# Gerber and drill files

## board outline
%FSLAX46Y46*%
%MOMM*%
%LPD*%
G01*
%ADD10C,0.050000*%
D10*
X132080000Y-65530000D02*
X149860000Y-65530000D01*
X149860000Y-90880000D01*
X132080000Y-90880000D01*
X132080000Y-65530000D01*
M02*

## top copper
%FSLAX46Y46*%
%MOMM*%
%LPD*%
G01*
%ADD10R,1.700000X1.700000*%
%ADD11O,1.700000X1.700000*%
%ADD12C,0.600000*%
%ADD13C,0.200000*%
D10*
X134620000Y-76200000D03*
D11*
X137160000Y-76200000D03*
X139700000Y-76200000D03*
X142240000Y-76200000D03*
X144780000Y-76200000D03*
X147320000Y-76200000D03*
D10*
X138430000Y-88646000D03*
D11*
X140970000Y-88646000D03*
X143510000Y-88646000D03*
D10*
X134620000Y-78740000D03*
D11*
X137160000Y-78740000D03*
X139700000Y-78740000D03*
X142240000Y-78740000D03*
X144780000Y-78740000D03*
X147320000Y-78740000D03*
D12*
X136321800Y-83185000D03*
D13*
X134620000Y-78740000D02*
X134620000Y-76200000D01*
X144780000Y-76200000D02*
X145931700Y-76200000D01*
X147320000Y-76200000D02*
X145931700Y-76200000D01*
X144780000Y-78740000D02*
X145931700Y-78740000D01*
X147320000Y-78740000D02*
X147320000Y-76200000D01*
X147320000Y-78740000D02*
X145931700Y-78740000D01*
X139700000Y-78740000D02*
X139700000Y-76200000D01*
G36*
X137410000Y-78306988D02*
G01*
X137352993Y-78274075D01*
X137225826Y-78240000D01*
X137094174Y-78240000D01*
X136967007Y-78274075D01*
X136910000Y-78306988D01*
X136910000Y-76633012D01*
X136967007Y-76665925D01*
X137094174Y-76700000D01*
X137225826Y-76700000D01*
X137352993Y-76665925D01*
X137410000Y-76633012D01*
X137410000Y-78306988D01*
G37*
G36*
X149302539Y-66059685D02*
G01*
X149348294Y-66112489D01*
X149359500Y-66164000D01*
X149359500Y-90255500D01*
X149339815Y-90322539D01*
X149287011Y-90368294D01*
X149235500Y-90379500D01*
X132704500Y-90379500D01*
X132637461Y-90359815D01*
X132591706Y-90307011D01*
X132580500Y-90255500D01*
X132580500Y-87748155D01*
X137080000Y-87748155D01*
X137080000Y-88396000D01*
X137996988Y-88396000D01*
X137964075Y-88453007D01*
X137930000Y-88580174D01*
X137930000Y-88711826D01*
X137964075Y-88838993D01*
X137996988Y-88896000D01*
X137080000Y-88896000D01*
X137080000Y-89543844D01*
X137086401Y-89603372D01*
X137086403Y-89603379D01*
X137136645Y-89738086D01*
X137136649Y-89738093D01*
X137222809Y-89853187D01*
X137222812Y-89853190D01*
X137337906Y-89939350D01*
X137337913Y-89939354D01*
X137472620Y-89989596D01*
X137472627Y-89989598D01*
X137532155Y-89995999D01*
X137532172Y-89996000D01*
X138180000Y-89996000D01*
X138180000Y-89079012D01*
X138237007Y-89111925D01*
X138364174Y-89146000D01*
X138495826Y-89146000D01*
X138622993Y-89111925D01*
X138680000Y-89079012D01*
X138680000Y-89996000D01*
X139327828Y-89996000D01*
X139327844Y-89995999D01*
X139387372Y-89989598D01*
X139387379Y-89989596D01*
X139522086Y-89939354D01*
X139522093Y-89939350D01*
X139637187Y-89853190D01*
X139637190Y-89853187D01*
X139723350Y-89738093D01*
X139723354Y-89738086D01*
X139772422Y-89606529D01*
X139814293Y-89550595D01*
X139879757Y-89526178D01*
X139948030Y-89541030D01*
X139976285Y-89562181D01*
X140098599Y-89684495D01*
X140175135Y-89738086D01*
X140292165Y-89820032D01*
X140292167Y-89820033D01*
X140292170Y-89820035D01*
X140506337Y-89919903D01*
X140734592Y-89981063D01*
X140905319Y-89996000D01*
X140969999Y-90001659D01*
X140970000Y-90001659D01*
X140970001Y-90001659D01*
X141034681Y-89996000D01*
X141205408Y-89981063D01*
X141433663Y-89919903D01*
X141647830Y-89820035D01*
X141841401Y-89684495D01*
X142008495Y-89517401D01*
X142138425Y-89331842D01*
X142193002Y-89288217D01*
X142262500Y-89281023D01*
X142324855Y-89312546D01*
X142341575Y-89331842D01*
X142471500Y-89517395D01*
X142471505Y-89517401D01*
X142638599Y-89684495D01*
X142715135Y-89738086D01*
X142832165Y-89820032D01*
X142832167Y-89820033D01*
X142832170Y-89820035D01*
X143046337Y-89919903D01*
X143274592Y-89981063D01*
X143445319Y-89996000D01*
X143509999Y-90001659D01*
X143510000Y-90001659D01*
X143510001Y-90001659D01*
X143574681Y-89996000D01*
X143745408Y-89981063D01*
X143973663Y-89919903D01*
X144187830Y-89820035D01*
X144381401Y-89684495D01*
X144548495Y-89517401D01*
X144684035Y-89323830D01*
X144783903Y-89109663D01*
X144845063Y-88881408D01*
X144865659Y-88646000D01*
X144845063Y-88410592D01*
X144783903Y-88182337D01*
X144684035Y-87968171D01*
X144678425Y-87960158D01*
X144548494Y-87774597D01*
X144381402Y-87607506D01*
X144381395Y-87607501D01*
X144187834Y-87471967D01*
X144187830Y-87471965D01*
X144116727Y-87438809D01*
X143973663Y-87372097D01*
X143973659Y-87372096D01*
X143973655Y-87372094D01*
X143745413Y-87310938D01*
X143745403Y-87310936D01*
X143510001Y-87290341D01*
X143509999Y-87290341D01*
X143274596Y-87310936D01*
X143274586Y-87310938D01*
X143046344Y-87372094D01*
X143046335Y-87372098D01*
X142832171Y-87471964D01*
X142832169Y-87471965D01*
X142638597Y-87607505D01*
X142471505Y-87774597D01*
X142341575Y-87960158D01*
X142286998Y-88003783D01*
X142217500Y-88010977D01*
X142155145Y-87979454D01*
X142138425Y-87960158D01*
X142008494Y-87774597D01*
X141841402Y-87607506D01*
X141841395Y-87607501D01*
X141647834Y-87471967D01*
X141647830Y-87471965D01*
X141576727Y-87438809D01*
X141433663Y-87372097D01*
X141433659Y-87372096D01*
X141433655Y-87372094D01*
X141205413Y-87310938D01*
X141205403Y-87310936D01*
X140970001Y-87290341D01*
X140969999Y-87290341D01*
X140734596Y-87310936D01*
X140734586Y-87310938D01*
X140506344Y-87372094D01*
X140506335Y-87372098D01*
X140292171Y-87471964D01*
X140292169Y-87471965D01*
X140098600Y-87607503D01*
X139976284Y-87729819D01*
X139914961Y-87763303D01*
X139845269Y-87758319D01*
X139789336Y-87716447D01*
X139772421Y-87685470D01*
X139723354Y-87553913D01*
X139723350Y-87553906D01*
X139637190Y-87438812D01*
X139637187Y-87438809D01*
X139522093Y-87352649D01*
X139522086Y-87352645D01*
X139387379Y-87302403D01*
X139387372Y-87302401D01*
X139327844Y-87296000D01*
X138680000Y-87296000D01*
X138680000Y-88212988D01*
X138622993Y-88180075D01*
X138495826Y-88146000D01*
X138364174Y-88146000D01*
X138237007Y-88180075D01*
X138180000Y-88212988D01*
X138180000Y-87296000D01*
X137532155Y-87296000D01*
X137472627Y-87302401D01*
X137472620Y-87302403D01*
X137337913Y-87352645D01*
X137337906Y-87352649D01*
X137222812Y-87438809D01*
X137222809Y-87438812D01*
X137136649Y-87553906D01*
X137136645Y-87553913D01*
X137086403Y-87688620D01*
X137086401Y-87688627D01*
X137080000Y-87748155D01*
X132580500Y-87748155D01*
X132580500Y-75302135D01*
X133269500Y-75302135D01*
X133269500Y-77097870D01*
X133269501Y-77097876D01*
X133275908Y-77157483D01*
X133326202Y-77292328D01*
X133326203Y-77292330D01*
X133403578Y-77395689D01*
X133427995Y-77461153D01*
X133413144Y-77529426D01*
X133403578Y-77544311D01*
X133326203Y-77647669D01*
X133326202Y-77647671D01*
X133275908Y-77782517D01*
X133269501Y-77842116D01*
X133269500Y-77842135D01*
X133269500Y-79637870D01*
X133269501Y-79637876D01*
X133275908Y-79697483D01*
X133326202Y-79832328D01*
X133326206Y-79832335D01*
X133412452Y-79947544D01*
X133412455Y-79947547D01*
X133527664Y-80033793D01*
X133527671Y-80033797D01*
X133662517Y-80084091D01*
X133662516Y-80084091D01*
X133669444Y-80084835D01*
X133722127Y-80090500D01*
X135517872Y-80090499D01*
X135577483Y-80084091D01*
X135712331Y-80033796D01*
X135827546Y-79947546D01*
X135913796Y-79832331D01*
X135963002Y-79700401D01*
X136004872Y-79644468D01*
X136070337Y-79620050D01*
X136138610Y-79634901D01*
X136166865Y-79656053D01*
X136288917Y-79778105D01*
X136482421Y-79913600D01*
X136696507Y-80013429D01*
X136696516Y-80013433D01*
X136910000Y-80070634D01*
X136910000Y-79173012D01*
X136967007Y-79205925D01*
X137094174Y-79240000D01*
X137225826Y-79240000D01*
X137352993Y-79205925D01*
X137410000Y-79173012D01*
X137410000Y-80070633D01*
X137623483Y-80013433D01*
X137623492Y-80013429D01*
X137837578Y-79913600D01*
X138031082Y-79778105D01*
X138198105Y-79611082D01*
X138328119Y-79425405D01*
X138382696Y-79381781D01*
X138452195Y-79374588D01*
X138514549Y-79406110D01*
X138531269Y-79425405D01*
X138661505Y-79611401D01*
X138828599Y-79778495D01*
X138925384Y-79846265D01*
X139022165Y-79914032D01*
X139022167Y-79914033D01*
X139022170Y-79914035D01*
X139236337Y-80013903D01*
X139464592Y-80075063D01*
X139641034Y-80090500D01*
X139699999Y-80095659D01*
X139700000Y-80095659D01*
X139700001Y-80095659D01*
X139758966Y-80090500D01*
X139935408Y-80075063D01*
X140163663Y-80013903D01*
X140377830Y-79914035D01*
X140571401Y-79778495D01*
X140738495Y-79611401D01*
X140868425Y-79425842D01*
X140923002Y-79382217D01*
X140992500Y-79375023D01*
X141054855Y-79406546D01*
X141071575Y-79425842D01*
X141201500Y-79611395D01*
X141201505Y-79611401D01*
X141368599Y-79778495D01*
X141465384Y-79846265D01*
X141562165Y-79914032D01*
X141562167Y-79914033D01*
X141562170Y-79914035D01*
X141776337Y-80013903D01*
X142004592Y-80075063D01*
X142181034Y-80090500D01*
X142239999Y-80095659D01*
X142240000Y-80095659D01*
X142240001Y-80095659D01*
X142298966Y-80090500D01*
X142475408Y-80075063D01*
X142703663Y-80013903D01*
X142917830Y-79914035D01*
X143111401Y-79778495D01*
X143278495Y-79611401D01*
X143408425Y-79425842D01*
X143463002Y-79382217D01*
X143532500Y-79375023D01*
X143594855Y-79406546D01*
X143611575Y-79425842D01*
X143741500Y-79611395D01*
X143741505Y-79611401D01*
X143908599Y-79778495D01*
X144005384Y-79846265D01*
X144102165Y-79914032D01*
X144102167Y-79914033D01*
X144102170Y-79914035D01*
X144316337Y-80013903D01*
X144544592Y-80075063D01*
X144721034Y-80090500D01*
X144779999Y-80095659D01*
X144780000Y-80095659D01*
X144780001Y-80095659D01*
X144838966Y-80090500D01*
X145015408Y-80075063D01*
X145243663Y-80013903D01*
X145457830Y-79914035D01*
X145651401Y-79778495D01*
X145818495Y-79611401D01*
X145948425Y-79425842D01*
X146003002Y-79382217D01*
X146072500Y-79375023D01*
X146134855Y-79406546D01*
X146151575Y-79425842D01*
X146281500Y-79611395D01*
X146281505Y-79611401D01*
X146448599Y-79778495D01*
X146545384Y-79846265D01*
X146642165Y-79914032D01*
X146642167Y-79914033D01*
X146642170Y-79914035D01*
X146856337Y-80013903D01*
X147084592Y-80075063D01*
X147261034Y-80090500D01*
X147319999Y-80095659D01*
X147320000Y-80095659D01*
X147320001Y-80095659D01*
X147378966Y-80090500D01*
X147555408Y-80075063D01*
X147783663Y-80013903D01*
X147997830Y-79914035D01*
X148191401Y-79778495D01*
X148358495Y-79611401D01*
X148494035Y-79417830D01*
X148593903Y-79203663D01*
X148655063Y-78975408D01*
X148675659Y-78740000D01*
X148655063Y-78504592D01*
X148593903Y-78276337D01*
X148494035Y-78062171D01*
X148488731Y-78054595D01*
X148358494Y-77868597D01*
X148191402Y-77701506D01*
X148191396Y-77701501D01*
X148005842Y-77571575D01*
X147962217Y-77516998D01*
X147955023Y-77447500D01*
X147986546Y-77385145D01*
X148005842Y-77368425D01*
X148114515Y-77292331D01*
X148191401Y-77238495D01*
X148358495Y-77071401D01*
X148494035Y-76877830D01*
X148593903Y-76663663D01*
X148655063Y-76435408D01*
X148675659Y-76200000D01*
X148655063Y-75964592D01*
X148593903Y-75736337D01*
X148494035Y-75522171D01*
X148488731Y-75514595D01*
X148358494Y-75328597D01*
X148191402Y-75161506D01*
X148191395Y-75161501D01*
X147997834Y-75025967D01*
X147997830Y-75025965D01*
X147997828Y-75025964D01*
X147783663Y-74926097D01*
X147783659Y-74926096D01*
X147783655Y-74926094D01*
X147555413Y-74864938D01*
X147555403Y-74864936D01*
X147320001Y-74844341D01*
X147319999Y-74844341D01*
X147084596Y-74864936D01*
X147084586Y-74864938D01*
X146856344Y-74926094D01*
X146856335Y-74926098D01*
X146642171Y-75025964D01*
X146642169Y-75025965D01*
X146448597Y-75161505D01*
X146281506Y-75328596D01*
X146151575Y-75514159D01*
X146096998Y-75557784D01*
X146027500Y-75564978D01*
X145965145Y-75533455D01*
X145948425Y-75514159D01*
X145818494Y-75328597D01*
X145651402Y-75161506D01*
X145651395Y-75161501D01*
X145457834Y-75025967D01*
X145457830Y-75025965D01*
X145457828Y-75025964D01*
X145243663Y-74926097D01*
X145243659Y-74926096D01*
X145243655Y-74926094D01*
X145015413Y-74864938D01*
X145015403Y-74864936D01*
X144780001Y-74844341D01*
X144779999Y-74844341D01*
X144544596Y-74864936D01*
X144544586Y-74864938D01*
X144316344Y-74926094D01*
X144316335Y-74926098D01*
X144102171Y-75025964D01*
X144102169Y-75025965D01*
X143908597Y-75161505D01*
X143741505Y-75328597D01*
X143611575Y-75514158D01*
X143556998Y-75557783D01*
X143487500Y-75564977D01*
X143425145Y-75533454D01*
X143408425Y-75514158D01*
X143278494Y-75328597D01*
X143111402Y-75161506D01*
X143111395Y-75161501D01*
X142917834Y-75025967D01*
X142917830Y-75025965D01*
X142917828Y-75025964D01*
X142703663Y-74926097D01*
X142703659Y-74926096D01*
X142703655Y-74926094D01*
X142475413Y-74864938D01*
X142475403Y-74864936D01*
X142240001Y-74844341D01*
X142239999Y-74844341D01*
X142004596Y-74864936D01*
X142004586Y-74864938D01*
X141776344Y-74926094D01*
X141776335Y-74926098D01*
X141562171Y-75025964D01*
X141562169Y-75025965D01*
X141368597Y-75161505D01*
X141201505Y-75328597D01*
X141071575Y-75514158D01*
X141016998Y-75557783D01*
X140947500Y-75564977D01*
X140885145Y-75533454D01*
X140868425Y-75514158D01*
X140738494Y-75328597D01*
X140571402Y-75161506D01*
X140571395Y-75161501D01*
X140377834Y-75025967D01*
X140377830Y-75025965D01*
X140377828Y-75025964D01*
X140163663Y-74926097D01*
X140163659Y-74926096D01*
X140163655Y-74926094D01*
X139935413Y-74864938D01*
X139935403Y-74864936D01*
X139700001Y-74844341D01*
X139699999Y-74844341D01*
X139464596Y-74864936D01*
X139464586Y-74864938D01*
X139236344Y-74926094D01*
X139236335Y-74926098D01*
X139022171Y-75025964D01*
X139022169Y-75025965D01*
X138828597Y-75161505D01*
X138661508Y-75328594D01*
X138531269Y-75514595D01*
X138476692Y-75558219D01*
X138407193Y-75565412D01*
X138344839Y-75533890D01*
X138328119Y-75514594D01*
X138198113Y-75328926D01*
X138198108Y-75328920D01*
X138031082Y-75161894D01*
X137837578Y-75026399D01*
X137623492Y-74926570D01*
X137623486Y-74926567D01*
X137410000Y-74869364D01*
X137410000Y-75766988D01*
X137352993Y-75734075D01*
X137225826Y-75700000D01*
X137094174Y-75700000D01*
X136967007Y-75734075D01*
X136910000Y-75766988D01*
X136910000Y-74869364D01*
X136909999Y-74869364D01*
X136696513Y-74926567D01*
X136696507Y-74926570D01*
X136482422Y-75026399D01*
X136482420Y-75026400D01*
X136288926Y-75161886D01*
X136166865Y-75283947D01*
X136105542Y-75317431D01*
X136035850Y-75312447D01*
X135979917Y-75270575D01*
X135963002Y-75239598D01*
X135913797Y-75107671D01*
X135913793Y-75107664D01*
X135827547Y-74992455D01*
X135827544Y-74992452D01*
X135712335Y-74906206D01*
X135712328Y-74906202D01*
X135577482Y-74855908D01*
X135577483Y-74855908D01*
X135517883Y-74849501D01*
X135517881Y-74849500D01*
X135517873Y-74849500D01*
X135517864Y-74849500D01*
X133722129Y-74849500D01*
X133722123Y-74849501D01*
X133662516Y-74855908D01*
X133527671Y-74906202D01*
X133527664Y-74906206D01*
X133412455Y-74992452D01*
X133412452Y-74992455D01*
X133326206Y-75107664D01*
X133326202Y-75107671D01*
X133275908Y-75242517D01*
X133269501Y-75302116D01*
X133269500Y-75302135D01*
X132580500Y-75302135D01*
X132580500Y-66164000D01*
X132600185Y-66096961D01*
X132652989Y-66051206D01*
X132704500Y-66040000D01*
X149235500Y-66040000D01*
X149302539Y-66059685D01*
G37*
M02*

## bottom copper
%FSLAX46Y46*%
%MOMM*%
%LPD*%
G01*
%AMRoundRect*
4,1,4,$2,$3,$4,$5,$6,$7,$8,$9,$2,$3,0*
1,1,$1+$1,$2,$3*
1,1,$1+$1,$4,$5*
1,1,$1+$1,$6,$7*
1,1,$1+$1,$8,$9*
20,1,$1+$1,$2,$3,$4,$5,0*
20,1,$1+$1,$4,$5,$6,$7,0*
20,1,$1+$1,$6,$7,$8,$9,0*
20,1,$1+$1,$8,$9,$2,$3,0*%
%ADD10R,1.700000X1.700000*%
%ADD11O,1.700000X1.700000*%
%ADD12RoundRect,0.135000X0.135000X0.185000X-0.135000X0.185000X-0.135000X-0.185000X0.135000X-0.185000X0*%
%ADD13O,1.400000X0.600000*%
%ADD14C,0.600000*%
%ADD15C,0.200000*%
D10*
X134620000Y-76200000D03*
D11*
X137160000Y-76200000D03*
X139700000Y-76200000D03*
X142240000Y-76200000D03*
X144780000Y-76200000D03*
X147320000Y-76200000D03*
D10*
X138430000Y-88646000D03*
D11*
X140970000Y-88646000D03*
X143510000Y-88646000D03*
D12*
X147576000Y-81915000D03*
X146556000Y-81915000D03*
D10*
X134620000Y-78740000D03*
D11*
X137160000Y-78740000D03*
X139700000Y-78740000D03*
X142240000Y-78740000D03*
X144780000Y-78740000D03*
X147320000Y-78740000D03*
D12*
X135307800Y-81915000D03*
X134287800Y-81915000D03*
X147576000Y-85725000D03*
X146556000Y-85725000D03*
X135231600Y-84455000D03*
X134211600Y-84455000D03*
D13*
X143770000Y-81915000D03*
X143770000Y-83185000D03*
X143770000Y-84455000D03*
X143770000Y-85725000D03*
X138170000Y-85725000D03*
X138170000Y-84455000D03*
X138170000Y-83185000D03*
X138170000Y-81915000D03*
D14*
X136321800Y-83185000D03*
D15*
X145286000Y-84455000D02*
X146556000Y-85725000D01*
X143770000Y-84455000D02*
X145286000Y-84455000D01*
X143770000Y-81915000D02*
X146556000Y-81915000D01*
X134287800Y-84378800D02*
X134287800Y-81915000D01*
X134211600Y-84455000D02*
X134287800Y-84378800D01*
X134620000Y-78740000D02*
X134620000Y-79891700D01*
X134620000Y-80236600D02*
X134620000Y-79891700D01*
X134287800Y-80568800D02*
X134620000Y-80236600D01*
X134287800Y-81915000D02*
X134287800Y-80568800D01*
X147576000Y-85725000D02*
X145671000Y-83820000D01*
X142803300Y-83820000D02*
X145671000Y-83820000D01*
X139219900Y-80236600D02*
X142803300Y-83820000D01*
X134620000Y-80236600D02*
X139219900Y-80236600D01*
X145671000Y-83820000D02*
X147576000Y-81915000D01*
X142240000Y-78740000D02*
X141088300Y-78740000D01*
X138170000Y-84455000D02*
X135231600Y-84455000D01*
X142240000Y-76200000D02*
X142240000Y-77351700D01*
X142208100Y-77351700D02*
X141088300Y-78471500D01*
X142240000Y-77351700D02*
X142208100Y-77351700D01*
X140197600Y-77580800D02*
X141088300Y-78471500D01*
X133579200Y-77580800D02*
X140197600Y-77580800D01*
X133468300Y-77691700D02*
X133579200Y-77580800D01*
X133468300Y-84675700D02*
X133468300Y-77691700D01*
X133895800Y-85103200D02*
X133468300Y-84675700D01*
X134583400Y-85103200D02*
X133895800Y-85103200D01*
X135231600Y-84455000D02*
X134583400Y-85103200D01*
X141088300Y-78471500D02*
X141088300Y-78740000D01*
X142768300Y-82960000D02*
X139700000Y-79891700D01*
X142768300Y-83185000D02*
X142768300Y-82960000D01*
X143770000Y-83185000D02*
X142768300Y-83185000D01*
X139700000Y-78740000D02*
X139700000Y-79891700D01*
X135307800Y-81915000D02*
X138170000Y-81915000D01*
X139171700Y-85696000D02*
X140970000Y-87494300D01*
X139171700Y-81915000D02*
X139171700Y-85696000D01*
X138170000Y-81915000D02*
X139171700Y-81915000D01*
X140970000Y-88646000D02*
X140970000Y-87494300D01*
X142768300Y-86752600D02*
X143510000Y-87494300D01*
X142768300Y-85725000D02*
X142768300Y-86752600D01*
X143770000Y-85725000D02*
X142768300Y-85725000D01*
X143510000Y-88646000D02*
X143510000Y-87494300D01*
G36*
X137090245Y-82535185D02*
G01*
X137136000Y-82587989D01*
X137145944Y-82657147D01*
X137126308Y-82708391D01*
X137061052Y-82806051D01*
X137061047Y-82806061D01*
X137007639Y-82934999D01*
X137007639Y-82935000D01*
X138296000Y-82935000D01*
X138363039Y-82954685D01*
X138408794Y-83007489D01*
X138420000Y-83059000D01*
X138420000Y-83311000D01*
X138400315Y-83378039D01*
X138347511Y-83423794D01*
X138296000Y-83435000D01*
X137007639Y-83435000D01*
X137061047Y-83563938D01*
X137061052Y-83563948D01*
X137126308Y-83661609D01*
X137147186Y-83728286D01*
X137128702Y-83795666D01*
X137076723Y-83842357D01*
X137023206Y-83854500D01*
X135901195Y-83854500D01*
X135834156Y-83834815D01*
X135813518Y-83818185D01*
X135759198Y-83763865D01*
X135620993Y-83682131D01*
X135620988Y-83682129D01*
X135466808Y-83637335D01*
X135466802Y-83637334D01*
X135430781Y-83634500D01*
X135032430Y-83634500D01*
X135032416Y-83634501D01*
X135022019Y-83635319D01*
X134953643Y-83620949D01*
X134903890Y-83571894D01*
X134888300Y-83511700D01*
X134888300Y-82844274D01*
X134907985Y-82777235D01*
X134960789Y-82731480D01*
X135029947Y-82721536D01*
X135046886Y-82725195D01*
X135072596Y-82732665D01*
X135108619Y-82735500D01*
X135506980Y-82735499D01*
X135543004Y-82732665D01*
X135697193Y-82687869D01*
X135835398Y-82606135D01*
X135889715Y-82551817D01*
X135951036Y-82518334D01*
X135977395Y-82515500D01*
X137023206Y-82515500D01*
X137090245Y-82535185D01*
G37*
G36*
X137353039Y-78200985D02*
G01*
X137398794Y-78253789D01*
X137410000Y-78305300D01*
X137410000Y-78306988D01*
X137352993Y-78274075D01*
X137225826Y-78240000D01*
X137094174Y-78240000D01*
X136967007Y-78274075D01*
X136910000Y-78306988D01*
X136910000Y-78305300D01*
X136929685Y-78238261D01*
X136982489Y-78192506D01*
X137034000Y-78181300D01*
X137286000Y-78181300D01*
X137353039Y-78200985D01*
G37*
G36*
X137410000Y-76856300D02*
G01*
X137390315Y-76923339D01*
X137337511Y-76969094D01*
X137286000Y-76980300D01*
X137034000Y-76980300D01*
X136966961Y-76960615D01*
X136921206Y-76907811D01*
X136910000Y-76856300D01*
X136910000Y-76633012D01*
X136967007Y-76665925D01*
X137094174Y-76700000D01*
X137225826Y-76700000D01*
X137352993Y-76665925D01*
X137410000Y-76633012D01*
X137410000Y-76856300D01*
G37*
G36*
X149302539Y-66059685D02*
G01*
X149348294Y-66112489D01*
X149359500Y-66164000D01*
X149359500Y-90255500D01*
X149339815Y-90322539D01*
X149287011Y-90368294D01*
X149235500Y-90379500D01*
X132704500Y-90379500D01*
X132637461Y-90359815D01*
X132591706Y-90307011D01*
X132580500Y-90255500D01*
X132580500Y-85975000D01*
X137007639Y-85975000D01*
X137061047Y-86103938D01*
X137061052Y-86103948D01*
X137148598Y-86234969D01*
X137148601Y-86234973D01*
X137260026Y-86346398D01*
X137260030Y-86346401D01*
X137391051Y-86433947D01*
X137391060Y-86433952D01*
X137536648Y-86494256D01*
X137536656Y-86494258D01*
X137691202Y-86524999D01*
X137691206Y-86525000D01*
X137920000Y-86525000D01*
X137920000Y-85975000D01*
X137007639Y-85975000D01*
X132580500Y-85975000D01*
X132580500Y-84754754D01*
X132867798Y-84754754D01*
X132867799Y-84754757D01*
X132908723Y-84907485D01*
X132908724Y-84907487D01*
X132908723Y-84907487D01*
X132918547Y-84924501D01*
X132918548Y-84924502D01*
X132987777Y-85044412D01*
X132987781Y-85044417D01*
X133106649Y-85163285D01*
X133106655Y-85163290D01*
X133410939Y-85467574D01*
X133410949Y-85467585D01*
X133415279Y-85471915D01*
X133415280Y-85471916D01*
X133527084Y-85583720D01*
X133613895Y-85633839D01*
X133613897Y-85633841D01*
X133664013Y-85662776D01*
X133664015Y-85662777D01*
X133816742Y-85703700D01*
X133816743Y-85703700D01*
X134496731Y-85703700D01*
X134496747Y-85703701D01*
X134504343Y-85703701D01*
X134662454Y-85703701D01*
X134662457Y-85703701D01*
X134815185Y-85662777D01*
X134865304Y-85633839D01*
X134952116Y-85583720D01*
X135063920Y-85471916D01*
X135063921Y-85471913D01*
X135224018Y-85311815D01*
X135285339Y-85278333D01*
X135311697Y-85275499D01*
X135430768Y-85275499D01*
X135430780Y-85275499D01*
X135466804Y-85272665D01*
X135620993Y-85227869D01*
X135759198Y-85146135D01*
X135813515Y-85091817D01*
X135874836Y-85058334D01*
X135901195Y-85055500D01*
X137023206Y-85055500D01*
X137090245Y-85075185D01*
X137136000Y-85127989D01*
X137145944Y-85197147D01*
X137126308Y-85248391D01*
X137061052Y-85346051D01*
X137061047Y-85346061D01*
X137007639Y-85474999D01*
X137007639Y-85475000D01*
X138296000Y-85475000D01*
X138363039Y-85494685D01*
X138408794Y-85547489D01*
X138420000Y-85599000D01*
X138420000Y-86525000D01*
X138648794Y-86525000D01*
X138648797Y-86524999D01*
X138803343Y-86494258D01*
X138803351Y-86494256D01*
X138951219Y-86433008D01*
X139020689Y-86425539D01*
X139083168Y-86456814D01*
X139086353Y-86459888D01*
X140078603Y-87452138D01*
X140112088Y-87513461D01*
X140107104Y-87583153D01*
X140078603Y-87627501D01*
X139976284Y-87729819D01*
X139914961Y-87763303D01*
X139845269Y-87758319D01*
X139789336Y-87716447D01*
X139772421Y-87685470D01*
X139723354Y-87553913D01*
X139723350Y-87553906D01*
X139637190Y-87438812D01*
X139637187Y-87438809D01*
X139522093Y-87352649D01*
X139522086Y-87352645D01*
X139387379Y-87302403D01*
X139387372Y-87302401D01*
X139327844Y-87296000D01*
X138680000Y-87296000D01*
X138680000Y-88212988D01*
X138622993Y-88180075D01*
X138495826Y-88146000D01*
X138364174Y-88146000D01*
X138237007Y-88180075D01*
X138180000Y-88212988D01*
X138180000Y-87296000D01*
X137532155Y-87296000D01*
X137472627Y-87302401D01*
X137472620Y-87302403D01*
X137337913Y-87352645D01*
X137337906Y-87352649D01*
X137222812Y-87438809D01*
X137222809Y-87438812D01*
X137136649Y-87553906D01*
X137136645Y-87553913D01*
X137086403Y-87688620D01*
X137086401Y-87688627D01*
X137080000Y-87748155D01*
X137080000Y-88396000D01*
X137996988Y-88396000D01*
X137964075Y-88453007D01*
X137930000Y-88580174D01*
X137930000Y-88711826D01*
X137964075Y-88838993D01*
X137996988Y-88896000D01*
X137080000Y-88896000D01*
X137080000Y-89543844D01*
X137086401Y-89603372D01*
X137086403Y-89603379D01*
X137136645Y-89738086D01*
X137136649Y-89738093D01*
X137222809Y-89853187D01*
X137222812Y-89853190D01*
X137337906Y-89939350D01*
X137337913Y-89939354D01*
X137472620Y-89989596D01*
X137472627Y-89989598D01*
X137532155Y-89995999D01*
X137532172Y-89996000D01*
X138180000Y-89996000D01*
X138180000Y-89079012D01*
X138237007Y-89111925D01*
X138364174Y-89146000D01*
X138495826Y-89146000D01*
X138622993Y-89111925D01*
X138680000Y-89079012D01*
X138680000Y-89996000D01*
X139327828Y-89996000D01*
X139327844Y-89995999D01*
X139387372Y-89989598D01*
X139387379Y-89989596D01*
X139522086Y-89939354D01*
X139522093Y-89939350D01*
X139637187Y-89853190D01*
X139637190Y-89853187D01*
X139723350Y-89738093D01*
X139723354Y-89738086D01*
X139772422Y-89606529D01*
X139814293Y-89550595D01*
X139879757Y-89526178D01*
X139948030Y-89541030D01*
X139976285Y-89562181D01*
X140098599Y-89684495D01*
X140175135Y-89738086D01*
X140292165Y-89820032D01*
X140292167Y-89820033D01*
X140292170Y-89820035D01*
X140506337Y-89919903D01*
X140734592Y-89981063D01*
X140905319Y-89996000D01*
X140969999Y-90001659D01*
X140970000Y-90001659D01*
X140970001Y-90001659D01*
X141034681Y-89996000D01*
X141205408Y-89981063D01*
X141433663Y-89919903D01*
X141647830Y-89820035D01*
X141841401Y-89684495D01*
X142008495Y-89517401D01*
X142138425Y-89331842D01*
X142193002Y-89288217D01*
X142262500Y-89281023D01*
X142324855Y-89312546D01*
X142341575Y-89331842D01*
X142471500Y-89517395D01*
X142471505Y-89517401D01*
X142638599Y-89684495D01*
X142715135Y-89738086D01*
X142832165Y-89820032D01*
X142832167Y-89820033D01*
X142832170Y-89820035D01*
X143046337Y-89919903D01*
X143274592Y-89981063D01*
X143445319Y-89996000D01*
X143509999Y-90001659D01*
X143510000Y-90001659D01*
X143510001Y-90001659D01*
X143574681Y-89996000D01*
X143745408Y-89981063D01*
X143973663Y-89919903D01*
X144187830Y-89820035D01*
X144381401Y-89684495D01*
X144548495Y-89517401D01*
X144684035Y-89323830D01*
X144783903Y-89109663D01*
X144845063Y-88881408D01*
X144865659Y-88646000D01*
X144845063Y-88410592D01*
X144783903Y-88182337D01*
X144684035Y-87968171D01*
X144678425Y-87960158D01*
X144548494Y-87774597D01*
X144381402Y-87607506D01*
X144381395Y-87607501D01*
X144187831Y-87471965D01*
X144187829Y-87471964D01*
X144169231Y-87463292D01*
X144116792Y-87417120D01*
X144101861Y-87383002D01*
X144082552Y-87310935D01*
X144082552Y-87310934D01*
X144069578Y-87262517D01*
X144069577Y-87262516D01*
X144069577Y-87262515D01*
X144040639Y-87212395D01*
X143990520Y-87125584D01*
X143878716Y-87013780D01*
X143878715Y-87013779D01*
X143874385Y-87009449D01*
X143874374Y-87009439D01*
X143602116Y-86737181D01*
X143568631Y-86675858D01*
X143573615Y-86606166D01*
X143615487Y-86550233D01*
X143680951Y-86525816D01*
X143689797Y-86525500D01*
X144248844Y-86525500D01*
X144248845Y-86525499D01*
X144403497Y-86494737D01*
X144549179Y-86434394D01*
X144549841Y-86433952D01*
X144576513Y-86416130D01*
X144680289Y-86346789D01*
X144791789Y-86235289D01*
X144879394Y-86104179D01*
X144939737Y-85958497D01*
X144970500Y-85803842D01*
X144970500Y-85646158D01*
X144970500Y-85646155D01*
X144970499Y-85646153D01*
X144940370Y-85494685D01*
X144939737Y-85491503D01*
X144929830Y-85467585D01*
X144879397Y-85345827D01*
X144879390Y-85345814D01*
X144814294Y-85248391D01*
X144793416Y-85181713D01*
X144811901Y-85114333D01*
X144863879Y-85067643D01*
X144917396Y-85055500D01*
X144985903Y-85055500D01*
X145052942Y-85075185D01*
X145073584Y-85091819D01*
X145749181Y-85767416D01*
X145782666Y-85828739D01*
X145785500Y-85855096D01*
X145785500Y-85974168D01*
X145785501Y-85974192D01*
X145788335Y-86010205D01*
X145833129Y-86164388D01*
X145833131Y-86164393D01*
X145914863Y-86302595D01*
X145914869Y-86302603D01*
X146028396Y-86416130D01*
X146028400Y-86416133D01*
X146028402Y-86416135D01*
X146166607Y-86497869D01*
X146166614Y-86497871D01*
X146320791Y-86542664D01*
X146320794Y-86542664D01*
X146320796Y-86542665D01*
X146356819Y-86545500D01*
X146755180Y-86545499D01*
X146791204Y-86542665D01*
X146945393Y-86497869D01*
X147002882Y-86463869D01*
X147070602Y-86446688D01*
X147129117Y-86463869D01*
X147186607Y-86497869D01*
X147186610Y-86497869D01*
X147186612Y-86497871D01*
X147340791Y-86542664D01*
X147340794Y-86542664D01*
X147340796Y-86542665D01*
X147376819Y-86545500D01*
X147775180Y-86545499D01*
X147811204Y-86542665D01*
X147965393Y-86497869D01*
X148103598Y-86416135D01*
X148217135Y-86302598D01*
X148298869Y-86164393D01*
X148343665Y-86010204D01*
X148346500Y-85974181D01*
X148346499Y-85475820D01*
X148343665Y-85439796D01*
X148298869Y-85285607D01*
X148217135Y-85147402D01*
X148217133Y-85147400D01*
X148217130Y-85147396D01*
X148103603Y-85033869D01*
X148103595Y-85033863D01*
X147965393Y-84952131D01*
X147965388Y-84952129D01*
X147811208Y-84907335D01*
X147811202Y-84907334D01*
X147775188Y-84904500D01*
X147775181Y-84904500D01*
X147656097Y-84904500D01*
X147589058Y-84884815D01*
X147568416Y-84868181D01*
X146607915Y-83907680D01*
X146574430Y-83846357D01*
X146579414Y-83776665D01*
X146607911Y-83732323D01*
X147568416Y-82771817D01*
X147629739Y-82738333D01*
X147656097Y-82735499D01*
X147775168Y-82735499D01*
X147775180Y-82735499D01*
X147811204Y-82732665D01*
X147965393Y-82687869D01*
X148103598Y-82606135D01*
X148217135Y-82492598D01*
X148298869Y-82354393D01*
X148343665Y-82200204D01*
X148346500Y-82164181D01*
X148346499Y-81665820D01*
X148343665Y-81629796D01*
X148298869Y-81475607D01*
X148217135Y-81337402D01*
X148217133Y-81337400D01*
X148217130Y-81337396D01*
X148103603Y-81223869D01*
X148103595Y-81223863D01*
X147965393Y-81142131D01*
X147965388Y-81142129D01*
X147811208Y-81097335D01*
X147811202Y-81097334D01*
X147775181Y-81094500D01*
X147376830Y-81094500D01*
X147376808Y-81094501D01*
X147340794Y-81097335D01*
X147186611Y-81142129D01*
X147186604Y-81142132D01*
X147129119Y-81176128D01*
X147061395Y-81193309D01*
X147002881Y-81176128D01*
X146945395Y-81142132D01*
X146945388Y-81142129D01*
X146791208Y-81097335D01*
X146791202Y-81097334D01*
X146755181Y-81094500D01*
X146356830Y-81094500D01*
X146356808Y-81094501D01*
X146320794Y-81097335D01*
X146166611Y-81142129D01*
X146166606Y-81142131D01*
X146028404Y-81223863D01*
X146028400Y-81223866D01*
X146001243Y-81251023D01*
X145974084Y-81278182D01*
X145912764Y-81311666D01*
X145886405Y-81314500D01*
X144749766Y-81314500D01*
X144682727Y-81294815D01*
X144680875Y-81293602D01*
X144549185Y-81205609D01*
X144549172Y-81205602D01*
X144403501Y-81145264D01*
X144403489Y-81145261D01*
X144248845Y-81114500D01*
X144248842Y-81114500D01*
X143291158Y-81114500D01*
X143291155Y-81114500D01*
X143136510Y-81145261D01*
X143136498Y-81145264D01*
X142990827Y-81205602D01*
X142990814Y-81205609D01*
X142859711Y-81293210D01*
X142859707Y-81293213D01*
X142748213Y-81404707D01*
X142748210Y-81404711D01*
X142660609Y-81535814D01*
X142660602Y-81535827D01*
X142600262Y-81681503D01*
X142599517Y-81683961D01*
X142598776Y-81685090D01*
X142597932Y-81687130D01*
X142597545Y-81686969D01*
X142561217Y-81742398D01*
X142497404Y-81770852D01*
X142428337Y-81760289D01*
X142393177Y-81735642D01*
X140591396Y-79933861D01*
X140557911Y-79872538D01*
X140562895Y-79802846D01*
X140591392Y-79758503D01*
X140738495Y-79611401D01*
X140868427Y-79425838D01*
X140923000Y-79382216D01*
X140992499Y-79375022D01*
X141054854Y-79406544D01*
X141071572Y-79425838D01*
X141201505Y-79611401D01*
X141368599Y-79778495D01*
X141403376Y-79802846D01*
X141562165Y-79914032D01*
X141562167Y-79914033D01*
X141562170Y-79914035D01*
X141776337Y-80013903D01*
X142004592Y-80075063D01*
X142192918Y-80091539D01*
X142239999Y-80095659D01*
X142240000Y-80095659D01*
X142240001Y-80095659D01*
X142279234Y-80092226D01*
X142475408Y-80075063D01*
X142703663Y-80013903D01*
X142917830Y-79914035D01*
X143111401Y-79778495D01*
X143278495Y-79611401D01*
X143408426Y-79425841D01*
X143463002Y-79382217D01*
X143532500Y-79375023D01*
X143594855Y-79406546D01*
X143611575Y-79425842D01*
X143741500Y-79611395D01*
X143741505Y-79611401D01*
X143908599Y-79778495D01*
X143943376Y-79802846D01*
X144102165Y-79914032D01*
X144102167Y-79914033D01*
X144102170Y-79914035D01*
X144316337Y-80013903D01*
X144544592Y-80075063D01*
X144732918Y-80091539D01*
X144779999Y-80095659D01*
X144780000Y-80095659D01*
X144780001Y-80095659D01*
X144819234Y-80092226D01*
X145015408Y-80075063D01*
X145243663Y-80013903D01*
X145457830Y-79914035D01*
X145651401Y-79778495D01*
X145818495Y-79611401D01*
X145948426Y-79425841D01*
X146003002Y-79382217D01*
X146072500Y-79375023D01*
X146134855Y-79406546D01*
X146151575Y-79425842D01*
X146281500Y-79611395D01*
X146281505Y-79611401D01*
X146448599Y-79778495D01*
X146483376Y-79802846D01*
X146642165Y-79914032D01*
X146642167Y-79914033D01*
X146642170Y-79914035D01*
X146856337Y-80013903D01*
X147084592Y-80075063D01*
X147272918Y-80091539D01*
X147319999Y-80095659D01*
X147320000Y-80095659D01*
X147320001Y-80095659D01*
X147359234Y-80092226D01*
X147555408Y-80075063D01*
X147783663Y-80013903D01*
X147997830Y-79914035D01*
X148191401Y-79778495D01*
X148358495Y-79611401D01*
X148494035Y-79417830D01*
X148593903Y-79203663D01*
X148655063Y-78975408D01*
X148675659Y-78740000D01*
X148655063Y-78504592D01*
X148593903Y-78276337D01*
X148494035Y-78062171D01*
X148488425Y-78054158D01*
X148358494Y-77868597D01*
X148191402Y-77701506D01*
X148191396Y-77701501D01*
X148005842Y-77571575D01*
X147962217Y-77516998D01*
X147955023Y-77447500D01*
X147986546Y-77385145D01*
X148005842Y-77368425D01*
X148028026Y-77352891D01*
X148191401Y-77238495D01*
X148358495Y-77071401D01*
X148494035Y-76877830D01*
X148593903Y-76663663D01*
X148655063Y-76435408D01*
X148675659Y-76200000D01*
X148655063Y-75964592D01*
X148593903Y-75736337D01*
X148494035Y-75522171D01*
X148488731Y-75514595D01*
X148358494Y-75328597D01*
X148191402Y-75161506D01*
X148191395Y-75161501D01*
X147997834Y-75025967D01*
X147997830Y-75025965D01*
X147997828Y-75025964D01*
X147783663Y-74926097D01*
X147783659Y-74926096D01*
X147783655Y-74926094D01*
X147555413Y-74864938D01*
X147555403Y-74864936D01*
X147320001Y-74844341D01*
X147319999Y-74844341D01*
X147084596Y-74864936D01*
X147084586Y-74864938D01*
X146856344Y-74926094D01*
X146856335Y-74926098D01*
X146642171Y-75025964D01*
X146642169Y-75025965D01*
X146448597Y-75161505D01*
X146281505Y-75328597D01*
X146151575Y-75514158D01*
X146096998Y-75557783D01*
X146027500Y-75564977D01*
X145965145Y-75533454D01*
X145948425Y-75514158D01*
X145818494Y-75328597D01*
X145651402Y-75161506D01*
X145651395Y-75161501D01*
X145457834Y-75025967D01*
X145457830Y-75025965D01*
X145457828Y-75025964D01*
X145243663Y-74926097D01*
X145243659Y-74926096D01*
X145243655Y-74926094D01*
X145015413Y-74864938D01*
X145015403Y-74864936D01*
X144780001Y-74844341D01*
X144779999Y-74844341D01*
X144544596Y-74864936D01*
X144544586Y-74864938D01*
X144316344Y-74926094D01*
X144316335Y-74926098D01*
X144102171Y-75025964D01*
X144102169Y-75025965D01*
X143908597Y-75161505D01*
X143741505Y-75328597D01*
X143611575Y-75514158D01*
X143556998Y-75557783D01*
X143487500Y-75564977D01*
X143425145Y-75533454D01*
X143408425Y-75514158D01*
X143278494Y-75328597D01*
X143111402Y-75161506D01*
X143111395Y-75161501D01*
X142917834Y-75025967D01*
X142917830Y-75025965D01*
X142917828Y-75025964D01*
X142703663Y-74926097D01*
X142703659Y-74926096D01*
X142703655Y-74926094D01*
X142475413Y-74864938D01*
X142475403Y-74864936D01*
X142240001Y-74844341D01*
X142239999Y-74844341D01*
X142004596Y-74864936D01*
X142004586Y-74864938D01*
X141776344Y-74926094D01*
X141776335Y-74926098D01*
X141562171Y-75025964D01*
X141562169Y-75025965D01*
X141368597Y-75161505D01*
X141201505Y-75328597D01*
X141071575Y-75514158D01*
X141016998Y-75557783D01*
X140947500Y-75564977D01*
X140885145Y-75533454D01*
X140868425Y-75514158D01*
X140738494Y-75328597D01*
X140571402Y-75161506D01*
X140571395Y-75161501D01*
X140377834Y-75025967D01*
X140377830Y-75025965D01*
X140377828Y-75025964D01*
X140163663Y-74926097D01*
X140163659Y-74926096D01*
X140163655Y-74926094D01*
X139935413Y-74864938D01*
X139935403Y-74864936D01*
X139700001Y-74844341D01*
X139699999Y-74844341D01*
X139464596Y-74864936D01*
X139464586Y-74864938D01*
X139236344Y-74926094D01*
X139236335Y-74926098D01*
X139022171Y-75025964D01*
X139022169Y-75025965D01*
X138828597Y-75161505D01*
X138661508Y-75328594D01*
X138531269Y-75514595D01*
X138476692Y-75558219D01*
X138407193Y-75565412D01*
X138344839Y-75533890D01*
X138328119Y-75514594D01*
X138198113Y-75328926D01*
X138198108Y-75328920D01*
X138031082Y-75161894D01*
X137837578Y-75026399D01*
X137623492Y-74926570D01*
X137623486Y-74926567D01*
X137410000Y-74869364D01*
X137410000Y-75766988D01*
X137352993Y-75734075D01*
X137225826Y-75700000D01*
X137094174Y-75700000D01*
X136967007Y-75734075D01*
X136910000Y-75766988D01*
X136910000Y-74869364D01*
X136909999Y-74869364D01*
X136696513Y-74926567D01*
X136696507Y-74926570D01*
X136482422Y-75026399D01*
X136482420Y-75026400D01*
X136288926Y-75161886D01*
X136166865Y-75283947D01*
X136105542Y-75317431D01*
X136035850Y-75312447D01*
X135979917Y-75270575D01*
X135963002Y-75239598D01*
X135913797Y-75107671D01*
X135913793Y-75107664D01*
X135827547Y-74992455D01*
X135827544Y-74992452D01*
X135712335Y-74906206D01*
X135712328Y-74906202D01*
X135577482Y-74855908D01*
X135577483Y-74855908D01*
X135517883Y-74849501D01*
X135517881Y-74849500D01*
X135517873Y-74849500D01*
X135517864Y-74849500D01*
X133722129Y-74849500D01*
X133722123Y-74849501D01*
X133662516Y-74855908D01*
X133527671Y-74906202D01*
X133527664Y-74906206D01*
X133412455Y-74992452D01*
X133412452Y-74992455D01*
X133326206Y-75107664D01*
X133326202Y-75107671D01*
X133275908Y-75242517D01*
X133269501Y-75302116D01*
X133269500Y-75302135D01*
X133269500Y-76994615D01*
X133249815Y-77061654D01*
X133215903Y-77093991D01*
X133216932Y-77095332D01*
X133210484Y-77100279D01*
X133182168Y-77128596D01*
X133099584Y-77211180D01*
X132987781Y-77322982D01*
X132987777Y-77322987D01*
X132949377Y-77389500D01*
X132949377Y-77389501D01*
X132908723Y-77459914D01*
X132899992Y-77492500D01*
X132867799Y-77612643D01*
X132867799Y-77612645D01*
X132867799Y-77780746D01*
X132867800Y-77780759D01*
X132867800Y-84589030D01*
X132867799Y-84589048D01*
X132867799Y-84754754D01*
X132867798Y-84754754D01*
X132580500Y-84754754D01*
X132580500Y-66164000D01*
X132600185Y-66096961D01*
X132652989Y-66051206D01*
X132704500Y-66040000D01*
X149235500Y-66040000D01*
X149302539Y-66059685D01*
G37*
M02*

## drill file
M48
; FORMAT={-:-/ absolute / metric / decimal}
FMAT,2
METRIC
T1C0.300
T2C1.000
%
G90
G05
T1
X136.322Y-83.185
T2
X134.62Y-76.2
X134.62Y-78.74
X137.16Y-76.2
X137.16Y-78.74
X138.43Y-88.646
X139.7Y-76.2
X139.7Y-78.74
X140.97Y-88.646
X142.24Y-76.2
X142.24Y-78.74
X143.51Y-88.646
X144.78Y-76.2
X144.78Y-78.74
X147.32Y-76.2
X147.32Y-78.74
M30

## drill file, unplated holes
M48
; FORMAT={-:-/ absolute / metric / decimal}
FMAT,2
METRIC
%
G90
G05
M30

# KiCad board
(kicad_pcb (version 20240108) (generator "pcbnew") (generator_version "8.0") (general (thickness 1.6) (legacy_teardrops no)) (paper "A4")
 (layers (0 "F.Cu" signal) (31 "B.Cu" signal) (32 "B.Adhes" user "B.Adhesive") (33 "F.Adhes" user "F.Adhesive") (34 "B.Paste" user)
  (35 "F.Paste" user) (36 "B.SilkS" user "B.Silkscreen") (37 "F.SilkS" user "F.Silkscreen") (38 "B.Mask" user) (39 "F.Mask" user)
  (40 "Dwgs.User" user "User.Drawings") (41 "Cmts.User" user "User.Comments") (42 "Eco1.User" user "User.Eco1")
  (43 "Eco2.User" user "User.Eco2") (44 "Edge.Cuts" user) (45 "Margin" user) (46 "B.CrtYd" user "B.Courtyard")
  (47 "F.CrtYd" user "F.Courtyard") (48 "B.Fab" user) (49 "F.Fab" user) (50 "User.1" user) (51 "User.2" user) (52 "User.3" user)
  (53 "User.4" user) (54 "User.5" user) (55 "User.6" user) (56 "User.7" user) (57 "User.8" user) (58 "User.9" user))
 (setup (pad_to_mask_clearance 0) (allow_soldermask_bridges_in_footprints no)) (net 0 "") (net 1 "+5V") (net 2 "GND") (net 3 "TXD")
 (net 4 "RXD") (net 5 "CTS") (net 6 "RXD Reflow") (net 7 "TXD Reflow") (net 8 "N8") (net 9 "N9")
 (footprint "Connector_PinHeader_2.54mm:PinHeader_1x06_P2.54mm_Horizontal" (layer "F.Cu") (at 134.62 76.2 90)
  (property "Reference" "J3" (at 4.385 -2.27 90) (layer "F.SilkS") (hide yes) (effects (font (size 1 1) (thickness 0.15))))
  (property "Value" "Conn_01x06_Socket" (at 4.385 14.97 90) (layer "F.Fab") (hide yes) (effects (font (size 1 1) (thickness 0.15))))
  (pad "1" thru_hole rect (at 0 0 90) (size 1.7 1.7) (drill 1) (layers "*.Cu" "*.Mask") (remove_unused_layers no) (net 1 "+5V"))
  (pad "2" thru_hole oval (at 0 2.54 90) (size 1.7 1.7) (drill 1) (layers "*.Cu" "*.Mask") (remove_unused_layers no) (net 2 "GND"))
  (pad "3" thru_hole oval (at 0 5.08 90) (size 1.7 1.7) (drill 1) (layers "*.Cu" "*.Mask") (remove_unused_layers no) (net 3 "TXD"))
  (pad "4" thru_hole oval (at 0 7.62 90) (size 1.7 1.7) (drill 1) (layers "*.Cu" "*.Mask") (remove_unused_layers no) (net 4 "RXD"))
  (pad "5" thru_hole oval (at 0 10.16 90) (size 1.7 1.7) (drill 1) (layers "*.Cu" "*.Mask") (remove_unused_layers no) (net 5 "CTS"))
  (pad "6" thru_hole oval (at 0 12.7 90) (size 1.7 1.7) (drill 1) (layers "*.Cu" "*.Mask") (remove_unused_layers no) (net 5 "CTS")))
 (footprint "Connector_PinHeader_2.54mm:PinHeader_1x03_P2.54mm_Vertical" (layer "F.Cu") (at 138.43 88.646 90)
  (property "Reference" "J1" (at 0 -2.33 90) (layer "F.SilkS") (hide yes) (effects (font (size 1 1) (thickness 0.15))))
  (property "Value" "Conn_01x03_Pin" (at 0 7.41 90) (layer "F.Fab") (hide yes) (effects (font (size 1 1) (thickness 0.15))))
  (pad "1" thru_hole rect (at 0 0 90) (size 1.7 1.7) (drill 1) (layers "*.Cu" "*.Mask") (remove_unused_layers no) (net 2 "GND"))
  (pad "2" thru_hole oval (at 0 2.54 90) (size 1.7 1.7) (drill 1) (layers "*.Cu" "*.Mask") (remove_unused_layers no) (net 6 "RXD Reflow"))
  (pad "3" thru_hole oval (at 0 5.08 90) (size 1.7 1.7) (drill 1) (layers "*.Cu" "*.Mask") (remove_unused_layers no) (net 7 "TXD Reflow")))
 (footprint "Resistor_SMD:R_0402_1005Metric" (layer "B.Cu") (at 147.066 81.915 180)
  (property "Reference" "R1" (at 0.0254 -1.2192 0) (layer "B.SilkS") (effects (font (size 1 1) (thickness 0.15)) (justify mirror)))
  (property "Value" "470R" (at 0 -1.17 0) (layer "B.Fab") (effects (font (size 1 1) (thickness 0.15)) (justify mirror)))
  (pad "1" smd roundrect (at -0.51 0 180) (size 0.54 0.64) (layers "B.Cu" "B.Paste" "B.Mask") (roundrect_rratio 0.25) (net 1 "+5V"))
  (pad "2" smd roundrect (at 0.51 0 180) (size 0.54 0.64) (layers "B.Cu" "B.Paste" "B.Mask") (roundrect_rratio 0.25) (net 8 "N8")))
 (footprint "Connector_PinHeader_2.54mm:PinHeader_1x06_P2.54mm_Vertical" (layer "B.Cu") (at 134.62 78.74 -90)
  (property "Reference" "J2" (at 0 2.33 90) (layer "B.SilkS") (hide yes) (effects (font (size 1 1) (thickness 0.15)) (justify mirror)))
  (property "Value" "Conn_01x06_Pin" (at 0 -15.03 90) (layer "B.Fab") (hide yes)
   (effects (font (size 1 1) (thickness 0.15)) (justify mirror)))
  (pad "1" thru_hole rect (at 0 0 270) (size 1.7 1.7) (drill 1) (layers "*.Cu" "*.Mask") (remove_unused_layers no) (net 1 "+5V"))
  (pad "2" thru_hole oval (at 0 -2.54 270) (size 1.7 1.7) (drill 1) (layers "*.Cu" "*.Mask") (remove_unused_layers no) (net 2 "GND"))
  (pad "3" thru_hole oval (at 0 -5.08 270) (size 1.7 1.7) (drill 1) (layers "*.Cu" "*.Mask") (remove_unused_layers no) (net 3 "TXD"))
  (pad "4" thru_hole oval (at 0 -7.62 270) (size 1.7 1.7) (drill 1) (layers "*.Cu" "*.Mask") (remove_unused_layers no) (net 4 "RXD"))
  (pad "5" thru_hole oval (at 0 -10.16 270) (size 1.7 1.7) (drill 1) (layers "*.Cu" "*.Mask") (remove_unused_layers no) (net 5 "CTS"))
  (pad "6" thru_hole oval (at 0 -12.7 270) (size 1.7 1.7) (drill 1) (layers "*.Cu" "*.Mask") (remove_unused_layers no) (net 5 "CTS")))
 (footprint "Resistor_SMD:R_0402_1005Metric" (layer "B.Cu") (at 134.7978 81.915 180)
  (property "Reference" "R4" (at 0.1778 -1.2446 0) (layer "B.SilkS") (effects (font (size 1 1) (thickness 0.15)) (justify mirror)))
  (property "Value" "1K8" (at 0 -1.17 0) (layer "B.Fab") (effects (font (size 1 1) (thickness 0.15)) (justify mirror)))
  (pad "1" smd roundrect (at -0.51 0 180) (size 0.54 0.64) (layers "B.Cu" "B.Paste" "B.Mask") (roundrect_rratio 0.25) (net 6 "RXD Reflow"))
  (pad "2" smd roundrect (at 0.51 0 180) (size 0.54 0.64) (layers "B.Cu" "B.Paste" "B.Mask") (roundrect_rratio 0.25) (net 1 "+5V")))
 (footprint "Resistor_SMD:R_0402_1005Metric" (layer "B.Cu") (at 147.066 85.725 180)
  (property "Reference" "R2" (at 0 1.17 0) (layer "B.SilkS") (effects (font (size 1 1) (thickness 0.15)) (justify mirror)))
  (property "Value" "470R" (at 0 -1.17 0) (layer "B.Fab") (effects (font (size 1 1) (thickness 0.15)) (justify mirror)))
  (pad "1" smd roundrect (at -0.51 0 180) (size 0.54 0.64) (layers "B.Cu" "B.Paste" "B.Mask") (roundrect_rratio 0.25) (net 1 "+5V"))
  (pad "2" smd roundrect (at 0.51 0 180) (size 0.54 0.64) (layers "B.Cu" "B.Paste" "B.Mask") (roundrect_rratio 0.25) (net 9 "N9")))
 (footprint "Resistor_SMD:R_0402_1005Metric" (layer "B.Cu") (at 134.7216 84.455 180)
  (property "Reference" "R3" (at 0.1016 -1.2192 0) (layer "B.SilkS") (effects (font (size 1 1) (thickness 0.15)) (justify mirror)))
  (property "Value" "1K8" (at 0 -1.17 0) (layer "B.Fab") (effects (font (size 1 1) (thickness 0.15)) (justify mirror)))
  (pad "1" smd roundrect (at -0.51 0 180) (size 0.54 0.64) (layers "B.Cu" "B.Paste" "B.Mask") (roundrect_rratio 0.25) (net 4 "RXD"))
  (pad "2" smd roundrect (at 0.51 0 180) (size 0.54 0.64) (layers "B.Cu" "B.Paste" "B.Mask") (roundrect_rratio 0.25) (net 1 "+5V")))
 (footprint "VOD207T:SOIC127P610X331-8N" (layer "B.Cu") (at 140.97 83.82 180)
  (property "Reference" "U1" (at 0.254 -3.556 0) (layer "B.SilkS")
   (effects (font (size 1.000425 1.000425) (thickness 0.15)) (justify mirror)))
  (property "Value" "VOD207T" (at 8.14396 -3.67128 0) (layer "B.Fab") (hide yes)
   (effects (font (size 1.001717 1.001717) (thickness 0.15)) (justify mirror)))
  (pad "1" smd oval (at -2.8 1.905 180) (size 1.4 0.6) (layers "B.Cu" "B.Paste" "B.Mask") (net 8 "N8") (solder_mask_margin 0.102))
  (pad "2" smd oval (at -2.8 0.635 180) (size 1.4 0.6) (layers "B.Cu" "B.Paste" "B.Mask") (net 3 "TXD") (solder_mask_margin 0.102))
  (pad "3" smd oval (at -2.8 -0.635 180) (size 1.4 0.6) (layers "B.Cu" "B.Paste" "B.Mask") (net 9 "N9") (solder_mask_margin 0.102))
  (pad "4" smd oval (at -2.8 -1.905 180) (size 1.4 0.6) (layers "B.Cu" "B.Paste" "B.Mask") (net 7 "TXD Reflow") (solder_mask_margin 0.102))
  (pad "5" smd oval (at 2.8 -1.905 180) (size 1.4 0.6) (layers "B.Cu" "B.Paste" "B.Mask") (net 2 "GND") (solder_mask_margin 0.102))
  (pad "6" smd oval (at 2.8 -0.635 180) (size 1.4 0.6) (layers "B.Cu" "B.Paste" "B.Mask") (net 4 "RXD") (solder_mask_margin 0.102))
  (pad "7" smd oval (at 2.8 0.635 180) (size 1.4 0.6) (layers "B.Cu" "B.Paste" "B.Mask") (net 2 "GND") (solder_mask_margin 0.102))
  (pad "8" smd oval (at 2.8 1.905 180) (size 1.4 0.6) (layers "B.Cu" "B.Paste" "B.Mask") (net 6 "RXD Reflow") (solder_mask_margin 0.102)))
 (gr_rect (start 132.08 65.53) (end 149.86 90.88) (stroke (width 0.05) (type default)) (fill none) (layer "Edge.Cuts"))
 (via (at 136.3218 83.185) (size 0.6) (drill 0.3) (layers "F.Cu" "B.Cu") (free yes) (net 2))
 (segment (start 143.51 88.646) (end 143.51 87.4943) (width 0.2) (layer "B.Cu") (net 7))
 (segment (start 143.77 85.725) (end 142.7683 85.725) (width 0.2) (layer "B.Cu") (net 7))
 (segment (start 142.7683 86.7526) (end 143.51 87.4943) (width 0.2) (layer "B.Cu") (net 7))
 (segment (start 142.7683 85.725) (end 142.7683 86.7526) (width 0.2) (layer "B.Cu") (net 7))
 (segment (start 138.17 81.915) (end 139.1717 81.915) (width 0.2) (layer "B.Cu") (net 6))
 (segment (start 139.1717 85.696) (end 140.97 87.4943) (width 0.2) (layer "B.Cu") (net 6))
 (segment (start 140.97 88.646) (end 140.97 87.4943) (width 0.2) (layer "B.Cu") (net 6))
 (segment (start 139.1717 81.915) (end 139.1717 85.696) (width 0.2) (layer "B.Cu") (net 6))
 (segment (start 135.3078 81.915) (end 138.17 81.915) (width 0.2) (layer "B.Cu") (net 6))
 (segment (start 139.7 78.74) (end 139.7 76.2) (width 0.2) (layer "F.Cu") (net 3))
 (segment (start 142.7683 82.96) (end 139.7 79.8917) (width 0.2) (layer "B.Cu") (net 3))
 (segment (start 143.77 83.185) (end 142.7683 83.185) (width 0.2) (layer "B.Cu") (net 3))
 (segment (start 139.7 78.74) (end 139.7 79.8917) (width 0.2) (layer "B.Cu") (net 3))
 (segment (start 142.7683 83.185) (end 142.7683 82.96) (width 0.2) (layer "B.Cu") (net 3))
 (segment (start 133.4683 77.6917) (end 133.5792 77.5808) (width 0.2) (layer "B.Cu") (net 4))
 (segment (start 134.5834 85.1032) (end 133.8958 85.1032) (width 0.2) (layer "B.Cu") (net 4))
 (segment (start 141.0883 78.4715) (end 141.0883 78.74) (width 0.2) (layer "B.Cu") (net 4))
 (segment (start 142.24 78.74) (end 141.0883 78.74) (width 0.2) (layer "B.Cu") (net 4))
 (segment (start 135.2316 84.455) (end 134.5834 85.1032) (width 0.2) (layer "B.Cu") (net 4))
 (segment (start 133.4683 84.6757) (end 133.4683 77.6917) (width 0.2) (layer "B.Cu") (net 4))
 (segment (start 142.24 76.2) (end 142.24 77.3517) (width 0.2) (layer "B.Cu") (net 4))
 (segment (start 133.8958 85.1032) (end 133.4683 84.6757) (width 0.2) (layer "B.Cu") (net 4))
 (segment (start 142.2081 77.3517) (end 141.0883 78.4715) (width 0.2) (layer "B.Cu") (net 4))
 (segment (start 133.5792 77.5808) (end 140.1976 77.5808) (width 0.2) (layer "B.Cu") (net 4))
 (segment (start 140.1976 77.5808) (end 141.0883 78.4715) (width 0.2) (layer "B.Cu") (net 4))
 (segment (start 138.17 84.455) (end 135.2316 84.455) (width 0.2) (layer "B.Cu") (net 4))
 (segment (start 142.24 77.3517) (end 142.2081 77.3517) (width 0.2) (layer "B.Cu") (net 4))
 (segment (start 147.32 78.74) (end 145.9317 78.74) (width 0.2) (layer "F.Cu") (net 5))
 (segment (start 144.78 76.2) (end 145.9317 76.2) (width 0.2) (layer "F.Cu") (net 5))
 (segment (start 147.32 78.74) (end 147.32 76.2) (width 0.2) (layer "F.Cu") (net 5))
 (segment (start 147.32 76.2) (end 145.9317 76.2) (width 0.2) (layer "F.Cu") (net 5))
 (segment (start 144.78 78.74) (end 145.9317 78.74) (width 0.2) (layer "F.Cu") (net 5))
 (segment (start 134.62 78.74) (end 134.62 76.2) (width 0.2) (layer "F.Cu") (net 1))
 (segment (start 134.62 80.2366) (end 139.2199 80.2366) (width 0.2) (layer "B.Cu") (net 1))
 (segment (start 134.2878 80.5688) (end 134.62 80.2366) (width 0.2) (layer "B.Cu") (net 1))
 (segment (start 147.576 85.725) (end 145.671 83.82) (width 0.2) (layer "B.Cu") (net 1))
 (segment (start 134.2116 84.455) (end 134.2878 84.3788) (width 0.2) (layer "B.Cu") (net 1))
 (segment (start 145.671 83.82) (end 147.576 81.915) (width 0.2) (layer "B.Cu") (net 1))
 (segment (start 134.62 78.74) (end 134.62 79.8917) (width 0.2) (layer "B.Cu") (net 1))
 (segment (start 134.2878 84.3788) (end 134.2878 81.915) (width 0.2) (layer "B.Cu") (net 1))
 (segment (start 142.8033 83.82) (end 145.671 83.82) (width 0.2) (layer "B.Cu") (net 1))
 (segment (start 134.62 80.2366) (end 134.62 79.8917) (width 0.2) (layer "B.Cu") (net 1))
 (segment (start 139.2199 80.2366) (end 142.8033 83.82) (width 0.2) (layer "B.Cu") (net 1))
 (segment (start 134.2878 81.915) (end 134.2878 80.5688) (width 0.2) (layer "B.Cu") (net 1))
 (segment (start 143.77 81.915) (end 146.556 81.915) (width 0.2) (layer "B.Cu") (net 8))
 (segment (start 145.286 84.455) (end 146.556 85.725) (width 0.2) (layer "B.Cu") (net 9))
 (segment (start 143.77 84.455) (end 145.286 84.455) (width 0.2) (layer "B.Cu") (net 9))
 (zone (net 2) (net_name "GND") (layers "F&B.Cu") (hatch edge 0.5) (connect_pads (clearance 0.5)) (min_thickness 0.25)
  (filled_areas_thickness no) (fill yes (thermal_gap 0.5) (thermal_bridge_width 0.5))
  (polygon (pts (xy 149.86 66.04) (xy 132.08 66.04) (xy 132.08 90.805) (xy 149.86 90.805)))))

